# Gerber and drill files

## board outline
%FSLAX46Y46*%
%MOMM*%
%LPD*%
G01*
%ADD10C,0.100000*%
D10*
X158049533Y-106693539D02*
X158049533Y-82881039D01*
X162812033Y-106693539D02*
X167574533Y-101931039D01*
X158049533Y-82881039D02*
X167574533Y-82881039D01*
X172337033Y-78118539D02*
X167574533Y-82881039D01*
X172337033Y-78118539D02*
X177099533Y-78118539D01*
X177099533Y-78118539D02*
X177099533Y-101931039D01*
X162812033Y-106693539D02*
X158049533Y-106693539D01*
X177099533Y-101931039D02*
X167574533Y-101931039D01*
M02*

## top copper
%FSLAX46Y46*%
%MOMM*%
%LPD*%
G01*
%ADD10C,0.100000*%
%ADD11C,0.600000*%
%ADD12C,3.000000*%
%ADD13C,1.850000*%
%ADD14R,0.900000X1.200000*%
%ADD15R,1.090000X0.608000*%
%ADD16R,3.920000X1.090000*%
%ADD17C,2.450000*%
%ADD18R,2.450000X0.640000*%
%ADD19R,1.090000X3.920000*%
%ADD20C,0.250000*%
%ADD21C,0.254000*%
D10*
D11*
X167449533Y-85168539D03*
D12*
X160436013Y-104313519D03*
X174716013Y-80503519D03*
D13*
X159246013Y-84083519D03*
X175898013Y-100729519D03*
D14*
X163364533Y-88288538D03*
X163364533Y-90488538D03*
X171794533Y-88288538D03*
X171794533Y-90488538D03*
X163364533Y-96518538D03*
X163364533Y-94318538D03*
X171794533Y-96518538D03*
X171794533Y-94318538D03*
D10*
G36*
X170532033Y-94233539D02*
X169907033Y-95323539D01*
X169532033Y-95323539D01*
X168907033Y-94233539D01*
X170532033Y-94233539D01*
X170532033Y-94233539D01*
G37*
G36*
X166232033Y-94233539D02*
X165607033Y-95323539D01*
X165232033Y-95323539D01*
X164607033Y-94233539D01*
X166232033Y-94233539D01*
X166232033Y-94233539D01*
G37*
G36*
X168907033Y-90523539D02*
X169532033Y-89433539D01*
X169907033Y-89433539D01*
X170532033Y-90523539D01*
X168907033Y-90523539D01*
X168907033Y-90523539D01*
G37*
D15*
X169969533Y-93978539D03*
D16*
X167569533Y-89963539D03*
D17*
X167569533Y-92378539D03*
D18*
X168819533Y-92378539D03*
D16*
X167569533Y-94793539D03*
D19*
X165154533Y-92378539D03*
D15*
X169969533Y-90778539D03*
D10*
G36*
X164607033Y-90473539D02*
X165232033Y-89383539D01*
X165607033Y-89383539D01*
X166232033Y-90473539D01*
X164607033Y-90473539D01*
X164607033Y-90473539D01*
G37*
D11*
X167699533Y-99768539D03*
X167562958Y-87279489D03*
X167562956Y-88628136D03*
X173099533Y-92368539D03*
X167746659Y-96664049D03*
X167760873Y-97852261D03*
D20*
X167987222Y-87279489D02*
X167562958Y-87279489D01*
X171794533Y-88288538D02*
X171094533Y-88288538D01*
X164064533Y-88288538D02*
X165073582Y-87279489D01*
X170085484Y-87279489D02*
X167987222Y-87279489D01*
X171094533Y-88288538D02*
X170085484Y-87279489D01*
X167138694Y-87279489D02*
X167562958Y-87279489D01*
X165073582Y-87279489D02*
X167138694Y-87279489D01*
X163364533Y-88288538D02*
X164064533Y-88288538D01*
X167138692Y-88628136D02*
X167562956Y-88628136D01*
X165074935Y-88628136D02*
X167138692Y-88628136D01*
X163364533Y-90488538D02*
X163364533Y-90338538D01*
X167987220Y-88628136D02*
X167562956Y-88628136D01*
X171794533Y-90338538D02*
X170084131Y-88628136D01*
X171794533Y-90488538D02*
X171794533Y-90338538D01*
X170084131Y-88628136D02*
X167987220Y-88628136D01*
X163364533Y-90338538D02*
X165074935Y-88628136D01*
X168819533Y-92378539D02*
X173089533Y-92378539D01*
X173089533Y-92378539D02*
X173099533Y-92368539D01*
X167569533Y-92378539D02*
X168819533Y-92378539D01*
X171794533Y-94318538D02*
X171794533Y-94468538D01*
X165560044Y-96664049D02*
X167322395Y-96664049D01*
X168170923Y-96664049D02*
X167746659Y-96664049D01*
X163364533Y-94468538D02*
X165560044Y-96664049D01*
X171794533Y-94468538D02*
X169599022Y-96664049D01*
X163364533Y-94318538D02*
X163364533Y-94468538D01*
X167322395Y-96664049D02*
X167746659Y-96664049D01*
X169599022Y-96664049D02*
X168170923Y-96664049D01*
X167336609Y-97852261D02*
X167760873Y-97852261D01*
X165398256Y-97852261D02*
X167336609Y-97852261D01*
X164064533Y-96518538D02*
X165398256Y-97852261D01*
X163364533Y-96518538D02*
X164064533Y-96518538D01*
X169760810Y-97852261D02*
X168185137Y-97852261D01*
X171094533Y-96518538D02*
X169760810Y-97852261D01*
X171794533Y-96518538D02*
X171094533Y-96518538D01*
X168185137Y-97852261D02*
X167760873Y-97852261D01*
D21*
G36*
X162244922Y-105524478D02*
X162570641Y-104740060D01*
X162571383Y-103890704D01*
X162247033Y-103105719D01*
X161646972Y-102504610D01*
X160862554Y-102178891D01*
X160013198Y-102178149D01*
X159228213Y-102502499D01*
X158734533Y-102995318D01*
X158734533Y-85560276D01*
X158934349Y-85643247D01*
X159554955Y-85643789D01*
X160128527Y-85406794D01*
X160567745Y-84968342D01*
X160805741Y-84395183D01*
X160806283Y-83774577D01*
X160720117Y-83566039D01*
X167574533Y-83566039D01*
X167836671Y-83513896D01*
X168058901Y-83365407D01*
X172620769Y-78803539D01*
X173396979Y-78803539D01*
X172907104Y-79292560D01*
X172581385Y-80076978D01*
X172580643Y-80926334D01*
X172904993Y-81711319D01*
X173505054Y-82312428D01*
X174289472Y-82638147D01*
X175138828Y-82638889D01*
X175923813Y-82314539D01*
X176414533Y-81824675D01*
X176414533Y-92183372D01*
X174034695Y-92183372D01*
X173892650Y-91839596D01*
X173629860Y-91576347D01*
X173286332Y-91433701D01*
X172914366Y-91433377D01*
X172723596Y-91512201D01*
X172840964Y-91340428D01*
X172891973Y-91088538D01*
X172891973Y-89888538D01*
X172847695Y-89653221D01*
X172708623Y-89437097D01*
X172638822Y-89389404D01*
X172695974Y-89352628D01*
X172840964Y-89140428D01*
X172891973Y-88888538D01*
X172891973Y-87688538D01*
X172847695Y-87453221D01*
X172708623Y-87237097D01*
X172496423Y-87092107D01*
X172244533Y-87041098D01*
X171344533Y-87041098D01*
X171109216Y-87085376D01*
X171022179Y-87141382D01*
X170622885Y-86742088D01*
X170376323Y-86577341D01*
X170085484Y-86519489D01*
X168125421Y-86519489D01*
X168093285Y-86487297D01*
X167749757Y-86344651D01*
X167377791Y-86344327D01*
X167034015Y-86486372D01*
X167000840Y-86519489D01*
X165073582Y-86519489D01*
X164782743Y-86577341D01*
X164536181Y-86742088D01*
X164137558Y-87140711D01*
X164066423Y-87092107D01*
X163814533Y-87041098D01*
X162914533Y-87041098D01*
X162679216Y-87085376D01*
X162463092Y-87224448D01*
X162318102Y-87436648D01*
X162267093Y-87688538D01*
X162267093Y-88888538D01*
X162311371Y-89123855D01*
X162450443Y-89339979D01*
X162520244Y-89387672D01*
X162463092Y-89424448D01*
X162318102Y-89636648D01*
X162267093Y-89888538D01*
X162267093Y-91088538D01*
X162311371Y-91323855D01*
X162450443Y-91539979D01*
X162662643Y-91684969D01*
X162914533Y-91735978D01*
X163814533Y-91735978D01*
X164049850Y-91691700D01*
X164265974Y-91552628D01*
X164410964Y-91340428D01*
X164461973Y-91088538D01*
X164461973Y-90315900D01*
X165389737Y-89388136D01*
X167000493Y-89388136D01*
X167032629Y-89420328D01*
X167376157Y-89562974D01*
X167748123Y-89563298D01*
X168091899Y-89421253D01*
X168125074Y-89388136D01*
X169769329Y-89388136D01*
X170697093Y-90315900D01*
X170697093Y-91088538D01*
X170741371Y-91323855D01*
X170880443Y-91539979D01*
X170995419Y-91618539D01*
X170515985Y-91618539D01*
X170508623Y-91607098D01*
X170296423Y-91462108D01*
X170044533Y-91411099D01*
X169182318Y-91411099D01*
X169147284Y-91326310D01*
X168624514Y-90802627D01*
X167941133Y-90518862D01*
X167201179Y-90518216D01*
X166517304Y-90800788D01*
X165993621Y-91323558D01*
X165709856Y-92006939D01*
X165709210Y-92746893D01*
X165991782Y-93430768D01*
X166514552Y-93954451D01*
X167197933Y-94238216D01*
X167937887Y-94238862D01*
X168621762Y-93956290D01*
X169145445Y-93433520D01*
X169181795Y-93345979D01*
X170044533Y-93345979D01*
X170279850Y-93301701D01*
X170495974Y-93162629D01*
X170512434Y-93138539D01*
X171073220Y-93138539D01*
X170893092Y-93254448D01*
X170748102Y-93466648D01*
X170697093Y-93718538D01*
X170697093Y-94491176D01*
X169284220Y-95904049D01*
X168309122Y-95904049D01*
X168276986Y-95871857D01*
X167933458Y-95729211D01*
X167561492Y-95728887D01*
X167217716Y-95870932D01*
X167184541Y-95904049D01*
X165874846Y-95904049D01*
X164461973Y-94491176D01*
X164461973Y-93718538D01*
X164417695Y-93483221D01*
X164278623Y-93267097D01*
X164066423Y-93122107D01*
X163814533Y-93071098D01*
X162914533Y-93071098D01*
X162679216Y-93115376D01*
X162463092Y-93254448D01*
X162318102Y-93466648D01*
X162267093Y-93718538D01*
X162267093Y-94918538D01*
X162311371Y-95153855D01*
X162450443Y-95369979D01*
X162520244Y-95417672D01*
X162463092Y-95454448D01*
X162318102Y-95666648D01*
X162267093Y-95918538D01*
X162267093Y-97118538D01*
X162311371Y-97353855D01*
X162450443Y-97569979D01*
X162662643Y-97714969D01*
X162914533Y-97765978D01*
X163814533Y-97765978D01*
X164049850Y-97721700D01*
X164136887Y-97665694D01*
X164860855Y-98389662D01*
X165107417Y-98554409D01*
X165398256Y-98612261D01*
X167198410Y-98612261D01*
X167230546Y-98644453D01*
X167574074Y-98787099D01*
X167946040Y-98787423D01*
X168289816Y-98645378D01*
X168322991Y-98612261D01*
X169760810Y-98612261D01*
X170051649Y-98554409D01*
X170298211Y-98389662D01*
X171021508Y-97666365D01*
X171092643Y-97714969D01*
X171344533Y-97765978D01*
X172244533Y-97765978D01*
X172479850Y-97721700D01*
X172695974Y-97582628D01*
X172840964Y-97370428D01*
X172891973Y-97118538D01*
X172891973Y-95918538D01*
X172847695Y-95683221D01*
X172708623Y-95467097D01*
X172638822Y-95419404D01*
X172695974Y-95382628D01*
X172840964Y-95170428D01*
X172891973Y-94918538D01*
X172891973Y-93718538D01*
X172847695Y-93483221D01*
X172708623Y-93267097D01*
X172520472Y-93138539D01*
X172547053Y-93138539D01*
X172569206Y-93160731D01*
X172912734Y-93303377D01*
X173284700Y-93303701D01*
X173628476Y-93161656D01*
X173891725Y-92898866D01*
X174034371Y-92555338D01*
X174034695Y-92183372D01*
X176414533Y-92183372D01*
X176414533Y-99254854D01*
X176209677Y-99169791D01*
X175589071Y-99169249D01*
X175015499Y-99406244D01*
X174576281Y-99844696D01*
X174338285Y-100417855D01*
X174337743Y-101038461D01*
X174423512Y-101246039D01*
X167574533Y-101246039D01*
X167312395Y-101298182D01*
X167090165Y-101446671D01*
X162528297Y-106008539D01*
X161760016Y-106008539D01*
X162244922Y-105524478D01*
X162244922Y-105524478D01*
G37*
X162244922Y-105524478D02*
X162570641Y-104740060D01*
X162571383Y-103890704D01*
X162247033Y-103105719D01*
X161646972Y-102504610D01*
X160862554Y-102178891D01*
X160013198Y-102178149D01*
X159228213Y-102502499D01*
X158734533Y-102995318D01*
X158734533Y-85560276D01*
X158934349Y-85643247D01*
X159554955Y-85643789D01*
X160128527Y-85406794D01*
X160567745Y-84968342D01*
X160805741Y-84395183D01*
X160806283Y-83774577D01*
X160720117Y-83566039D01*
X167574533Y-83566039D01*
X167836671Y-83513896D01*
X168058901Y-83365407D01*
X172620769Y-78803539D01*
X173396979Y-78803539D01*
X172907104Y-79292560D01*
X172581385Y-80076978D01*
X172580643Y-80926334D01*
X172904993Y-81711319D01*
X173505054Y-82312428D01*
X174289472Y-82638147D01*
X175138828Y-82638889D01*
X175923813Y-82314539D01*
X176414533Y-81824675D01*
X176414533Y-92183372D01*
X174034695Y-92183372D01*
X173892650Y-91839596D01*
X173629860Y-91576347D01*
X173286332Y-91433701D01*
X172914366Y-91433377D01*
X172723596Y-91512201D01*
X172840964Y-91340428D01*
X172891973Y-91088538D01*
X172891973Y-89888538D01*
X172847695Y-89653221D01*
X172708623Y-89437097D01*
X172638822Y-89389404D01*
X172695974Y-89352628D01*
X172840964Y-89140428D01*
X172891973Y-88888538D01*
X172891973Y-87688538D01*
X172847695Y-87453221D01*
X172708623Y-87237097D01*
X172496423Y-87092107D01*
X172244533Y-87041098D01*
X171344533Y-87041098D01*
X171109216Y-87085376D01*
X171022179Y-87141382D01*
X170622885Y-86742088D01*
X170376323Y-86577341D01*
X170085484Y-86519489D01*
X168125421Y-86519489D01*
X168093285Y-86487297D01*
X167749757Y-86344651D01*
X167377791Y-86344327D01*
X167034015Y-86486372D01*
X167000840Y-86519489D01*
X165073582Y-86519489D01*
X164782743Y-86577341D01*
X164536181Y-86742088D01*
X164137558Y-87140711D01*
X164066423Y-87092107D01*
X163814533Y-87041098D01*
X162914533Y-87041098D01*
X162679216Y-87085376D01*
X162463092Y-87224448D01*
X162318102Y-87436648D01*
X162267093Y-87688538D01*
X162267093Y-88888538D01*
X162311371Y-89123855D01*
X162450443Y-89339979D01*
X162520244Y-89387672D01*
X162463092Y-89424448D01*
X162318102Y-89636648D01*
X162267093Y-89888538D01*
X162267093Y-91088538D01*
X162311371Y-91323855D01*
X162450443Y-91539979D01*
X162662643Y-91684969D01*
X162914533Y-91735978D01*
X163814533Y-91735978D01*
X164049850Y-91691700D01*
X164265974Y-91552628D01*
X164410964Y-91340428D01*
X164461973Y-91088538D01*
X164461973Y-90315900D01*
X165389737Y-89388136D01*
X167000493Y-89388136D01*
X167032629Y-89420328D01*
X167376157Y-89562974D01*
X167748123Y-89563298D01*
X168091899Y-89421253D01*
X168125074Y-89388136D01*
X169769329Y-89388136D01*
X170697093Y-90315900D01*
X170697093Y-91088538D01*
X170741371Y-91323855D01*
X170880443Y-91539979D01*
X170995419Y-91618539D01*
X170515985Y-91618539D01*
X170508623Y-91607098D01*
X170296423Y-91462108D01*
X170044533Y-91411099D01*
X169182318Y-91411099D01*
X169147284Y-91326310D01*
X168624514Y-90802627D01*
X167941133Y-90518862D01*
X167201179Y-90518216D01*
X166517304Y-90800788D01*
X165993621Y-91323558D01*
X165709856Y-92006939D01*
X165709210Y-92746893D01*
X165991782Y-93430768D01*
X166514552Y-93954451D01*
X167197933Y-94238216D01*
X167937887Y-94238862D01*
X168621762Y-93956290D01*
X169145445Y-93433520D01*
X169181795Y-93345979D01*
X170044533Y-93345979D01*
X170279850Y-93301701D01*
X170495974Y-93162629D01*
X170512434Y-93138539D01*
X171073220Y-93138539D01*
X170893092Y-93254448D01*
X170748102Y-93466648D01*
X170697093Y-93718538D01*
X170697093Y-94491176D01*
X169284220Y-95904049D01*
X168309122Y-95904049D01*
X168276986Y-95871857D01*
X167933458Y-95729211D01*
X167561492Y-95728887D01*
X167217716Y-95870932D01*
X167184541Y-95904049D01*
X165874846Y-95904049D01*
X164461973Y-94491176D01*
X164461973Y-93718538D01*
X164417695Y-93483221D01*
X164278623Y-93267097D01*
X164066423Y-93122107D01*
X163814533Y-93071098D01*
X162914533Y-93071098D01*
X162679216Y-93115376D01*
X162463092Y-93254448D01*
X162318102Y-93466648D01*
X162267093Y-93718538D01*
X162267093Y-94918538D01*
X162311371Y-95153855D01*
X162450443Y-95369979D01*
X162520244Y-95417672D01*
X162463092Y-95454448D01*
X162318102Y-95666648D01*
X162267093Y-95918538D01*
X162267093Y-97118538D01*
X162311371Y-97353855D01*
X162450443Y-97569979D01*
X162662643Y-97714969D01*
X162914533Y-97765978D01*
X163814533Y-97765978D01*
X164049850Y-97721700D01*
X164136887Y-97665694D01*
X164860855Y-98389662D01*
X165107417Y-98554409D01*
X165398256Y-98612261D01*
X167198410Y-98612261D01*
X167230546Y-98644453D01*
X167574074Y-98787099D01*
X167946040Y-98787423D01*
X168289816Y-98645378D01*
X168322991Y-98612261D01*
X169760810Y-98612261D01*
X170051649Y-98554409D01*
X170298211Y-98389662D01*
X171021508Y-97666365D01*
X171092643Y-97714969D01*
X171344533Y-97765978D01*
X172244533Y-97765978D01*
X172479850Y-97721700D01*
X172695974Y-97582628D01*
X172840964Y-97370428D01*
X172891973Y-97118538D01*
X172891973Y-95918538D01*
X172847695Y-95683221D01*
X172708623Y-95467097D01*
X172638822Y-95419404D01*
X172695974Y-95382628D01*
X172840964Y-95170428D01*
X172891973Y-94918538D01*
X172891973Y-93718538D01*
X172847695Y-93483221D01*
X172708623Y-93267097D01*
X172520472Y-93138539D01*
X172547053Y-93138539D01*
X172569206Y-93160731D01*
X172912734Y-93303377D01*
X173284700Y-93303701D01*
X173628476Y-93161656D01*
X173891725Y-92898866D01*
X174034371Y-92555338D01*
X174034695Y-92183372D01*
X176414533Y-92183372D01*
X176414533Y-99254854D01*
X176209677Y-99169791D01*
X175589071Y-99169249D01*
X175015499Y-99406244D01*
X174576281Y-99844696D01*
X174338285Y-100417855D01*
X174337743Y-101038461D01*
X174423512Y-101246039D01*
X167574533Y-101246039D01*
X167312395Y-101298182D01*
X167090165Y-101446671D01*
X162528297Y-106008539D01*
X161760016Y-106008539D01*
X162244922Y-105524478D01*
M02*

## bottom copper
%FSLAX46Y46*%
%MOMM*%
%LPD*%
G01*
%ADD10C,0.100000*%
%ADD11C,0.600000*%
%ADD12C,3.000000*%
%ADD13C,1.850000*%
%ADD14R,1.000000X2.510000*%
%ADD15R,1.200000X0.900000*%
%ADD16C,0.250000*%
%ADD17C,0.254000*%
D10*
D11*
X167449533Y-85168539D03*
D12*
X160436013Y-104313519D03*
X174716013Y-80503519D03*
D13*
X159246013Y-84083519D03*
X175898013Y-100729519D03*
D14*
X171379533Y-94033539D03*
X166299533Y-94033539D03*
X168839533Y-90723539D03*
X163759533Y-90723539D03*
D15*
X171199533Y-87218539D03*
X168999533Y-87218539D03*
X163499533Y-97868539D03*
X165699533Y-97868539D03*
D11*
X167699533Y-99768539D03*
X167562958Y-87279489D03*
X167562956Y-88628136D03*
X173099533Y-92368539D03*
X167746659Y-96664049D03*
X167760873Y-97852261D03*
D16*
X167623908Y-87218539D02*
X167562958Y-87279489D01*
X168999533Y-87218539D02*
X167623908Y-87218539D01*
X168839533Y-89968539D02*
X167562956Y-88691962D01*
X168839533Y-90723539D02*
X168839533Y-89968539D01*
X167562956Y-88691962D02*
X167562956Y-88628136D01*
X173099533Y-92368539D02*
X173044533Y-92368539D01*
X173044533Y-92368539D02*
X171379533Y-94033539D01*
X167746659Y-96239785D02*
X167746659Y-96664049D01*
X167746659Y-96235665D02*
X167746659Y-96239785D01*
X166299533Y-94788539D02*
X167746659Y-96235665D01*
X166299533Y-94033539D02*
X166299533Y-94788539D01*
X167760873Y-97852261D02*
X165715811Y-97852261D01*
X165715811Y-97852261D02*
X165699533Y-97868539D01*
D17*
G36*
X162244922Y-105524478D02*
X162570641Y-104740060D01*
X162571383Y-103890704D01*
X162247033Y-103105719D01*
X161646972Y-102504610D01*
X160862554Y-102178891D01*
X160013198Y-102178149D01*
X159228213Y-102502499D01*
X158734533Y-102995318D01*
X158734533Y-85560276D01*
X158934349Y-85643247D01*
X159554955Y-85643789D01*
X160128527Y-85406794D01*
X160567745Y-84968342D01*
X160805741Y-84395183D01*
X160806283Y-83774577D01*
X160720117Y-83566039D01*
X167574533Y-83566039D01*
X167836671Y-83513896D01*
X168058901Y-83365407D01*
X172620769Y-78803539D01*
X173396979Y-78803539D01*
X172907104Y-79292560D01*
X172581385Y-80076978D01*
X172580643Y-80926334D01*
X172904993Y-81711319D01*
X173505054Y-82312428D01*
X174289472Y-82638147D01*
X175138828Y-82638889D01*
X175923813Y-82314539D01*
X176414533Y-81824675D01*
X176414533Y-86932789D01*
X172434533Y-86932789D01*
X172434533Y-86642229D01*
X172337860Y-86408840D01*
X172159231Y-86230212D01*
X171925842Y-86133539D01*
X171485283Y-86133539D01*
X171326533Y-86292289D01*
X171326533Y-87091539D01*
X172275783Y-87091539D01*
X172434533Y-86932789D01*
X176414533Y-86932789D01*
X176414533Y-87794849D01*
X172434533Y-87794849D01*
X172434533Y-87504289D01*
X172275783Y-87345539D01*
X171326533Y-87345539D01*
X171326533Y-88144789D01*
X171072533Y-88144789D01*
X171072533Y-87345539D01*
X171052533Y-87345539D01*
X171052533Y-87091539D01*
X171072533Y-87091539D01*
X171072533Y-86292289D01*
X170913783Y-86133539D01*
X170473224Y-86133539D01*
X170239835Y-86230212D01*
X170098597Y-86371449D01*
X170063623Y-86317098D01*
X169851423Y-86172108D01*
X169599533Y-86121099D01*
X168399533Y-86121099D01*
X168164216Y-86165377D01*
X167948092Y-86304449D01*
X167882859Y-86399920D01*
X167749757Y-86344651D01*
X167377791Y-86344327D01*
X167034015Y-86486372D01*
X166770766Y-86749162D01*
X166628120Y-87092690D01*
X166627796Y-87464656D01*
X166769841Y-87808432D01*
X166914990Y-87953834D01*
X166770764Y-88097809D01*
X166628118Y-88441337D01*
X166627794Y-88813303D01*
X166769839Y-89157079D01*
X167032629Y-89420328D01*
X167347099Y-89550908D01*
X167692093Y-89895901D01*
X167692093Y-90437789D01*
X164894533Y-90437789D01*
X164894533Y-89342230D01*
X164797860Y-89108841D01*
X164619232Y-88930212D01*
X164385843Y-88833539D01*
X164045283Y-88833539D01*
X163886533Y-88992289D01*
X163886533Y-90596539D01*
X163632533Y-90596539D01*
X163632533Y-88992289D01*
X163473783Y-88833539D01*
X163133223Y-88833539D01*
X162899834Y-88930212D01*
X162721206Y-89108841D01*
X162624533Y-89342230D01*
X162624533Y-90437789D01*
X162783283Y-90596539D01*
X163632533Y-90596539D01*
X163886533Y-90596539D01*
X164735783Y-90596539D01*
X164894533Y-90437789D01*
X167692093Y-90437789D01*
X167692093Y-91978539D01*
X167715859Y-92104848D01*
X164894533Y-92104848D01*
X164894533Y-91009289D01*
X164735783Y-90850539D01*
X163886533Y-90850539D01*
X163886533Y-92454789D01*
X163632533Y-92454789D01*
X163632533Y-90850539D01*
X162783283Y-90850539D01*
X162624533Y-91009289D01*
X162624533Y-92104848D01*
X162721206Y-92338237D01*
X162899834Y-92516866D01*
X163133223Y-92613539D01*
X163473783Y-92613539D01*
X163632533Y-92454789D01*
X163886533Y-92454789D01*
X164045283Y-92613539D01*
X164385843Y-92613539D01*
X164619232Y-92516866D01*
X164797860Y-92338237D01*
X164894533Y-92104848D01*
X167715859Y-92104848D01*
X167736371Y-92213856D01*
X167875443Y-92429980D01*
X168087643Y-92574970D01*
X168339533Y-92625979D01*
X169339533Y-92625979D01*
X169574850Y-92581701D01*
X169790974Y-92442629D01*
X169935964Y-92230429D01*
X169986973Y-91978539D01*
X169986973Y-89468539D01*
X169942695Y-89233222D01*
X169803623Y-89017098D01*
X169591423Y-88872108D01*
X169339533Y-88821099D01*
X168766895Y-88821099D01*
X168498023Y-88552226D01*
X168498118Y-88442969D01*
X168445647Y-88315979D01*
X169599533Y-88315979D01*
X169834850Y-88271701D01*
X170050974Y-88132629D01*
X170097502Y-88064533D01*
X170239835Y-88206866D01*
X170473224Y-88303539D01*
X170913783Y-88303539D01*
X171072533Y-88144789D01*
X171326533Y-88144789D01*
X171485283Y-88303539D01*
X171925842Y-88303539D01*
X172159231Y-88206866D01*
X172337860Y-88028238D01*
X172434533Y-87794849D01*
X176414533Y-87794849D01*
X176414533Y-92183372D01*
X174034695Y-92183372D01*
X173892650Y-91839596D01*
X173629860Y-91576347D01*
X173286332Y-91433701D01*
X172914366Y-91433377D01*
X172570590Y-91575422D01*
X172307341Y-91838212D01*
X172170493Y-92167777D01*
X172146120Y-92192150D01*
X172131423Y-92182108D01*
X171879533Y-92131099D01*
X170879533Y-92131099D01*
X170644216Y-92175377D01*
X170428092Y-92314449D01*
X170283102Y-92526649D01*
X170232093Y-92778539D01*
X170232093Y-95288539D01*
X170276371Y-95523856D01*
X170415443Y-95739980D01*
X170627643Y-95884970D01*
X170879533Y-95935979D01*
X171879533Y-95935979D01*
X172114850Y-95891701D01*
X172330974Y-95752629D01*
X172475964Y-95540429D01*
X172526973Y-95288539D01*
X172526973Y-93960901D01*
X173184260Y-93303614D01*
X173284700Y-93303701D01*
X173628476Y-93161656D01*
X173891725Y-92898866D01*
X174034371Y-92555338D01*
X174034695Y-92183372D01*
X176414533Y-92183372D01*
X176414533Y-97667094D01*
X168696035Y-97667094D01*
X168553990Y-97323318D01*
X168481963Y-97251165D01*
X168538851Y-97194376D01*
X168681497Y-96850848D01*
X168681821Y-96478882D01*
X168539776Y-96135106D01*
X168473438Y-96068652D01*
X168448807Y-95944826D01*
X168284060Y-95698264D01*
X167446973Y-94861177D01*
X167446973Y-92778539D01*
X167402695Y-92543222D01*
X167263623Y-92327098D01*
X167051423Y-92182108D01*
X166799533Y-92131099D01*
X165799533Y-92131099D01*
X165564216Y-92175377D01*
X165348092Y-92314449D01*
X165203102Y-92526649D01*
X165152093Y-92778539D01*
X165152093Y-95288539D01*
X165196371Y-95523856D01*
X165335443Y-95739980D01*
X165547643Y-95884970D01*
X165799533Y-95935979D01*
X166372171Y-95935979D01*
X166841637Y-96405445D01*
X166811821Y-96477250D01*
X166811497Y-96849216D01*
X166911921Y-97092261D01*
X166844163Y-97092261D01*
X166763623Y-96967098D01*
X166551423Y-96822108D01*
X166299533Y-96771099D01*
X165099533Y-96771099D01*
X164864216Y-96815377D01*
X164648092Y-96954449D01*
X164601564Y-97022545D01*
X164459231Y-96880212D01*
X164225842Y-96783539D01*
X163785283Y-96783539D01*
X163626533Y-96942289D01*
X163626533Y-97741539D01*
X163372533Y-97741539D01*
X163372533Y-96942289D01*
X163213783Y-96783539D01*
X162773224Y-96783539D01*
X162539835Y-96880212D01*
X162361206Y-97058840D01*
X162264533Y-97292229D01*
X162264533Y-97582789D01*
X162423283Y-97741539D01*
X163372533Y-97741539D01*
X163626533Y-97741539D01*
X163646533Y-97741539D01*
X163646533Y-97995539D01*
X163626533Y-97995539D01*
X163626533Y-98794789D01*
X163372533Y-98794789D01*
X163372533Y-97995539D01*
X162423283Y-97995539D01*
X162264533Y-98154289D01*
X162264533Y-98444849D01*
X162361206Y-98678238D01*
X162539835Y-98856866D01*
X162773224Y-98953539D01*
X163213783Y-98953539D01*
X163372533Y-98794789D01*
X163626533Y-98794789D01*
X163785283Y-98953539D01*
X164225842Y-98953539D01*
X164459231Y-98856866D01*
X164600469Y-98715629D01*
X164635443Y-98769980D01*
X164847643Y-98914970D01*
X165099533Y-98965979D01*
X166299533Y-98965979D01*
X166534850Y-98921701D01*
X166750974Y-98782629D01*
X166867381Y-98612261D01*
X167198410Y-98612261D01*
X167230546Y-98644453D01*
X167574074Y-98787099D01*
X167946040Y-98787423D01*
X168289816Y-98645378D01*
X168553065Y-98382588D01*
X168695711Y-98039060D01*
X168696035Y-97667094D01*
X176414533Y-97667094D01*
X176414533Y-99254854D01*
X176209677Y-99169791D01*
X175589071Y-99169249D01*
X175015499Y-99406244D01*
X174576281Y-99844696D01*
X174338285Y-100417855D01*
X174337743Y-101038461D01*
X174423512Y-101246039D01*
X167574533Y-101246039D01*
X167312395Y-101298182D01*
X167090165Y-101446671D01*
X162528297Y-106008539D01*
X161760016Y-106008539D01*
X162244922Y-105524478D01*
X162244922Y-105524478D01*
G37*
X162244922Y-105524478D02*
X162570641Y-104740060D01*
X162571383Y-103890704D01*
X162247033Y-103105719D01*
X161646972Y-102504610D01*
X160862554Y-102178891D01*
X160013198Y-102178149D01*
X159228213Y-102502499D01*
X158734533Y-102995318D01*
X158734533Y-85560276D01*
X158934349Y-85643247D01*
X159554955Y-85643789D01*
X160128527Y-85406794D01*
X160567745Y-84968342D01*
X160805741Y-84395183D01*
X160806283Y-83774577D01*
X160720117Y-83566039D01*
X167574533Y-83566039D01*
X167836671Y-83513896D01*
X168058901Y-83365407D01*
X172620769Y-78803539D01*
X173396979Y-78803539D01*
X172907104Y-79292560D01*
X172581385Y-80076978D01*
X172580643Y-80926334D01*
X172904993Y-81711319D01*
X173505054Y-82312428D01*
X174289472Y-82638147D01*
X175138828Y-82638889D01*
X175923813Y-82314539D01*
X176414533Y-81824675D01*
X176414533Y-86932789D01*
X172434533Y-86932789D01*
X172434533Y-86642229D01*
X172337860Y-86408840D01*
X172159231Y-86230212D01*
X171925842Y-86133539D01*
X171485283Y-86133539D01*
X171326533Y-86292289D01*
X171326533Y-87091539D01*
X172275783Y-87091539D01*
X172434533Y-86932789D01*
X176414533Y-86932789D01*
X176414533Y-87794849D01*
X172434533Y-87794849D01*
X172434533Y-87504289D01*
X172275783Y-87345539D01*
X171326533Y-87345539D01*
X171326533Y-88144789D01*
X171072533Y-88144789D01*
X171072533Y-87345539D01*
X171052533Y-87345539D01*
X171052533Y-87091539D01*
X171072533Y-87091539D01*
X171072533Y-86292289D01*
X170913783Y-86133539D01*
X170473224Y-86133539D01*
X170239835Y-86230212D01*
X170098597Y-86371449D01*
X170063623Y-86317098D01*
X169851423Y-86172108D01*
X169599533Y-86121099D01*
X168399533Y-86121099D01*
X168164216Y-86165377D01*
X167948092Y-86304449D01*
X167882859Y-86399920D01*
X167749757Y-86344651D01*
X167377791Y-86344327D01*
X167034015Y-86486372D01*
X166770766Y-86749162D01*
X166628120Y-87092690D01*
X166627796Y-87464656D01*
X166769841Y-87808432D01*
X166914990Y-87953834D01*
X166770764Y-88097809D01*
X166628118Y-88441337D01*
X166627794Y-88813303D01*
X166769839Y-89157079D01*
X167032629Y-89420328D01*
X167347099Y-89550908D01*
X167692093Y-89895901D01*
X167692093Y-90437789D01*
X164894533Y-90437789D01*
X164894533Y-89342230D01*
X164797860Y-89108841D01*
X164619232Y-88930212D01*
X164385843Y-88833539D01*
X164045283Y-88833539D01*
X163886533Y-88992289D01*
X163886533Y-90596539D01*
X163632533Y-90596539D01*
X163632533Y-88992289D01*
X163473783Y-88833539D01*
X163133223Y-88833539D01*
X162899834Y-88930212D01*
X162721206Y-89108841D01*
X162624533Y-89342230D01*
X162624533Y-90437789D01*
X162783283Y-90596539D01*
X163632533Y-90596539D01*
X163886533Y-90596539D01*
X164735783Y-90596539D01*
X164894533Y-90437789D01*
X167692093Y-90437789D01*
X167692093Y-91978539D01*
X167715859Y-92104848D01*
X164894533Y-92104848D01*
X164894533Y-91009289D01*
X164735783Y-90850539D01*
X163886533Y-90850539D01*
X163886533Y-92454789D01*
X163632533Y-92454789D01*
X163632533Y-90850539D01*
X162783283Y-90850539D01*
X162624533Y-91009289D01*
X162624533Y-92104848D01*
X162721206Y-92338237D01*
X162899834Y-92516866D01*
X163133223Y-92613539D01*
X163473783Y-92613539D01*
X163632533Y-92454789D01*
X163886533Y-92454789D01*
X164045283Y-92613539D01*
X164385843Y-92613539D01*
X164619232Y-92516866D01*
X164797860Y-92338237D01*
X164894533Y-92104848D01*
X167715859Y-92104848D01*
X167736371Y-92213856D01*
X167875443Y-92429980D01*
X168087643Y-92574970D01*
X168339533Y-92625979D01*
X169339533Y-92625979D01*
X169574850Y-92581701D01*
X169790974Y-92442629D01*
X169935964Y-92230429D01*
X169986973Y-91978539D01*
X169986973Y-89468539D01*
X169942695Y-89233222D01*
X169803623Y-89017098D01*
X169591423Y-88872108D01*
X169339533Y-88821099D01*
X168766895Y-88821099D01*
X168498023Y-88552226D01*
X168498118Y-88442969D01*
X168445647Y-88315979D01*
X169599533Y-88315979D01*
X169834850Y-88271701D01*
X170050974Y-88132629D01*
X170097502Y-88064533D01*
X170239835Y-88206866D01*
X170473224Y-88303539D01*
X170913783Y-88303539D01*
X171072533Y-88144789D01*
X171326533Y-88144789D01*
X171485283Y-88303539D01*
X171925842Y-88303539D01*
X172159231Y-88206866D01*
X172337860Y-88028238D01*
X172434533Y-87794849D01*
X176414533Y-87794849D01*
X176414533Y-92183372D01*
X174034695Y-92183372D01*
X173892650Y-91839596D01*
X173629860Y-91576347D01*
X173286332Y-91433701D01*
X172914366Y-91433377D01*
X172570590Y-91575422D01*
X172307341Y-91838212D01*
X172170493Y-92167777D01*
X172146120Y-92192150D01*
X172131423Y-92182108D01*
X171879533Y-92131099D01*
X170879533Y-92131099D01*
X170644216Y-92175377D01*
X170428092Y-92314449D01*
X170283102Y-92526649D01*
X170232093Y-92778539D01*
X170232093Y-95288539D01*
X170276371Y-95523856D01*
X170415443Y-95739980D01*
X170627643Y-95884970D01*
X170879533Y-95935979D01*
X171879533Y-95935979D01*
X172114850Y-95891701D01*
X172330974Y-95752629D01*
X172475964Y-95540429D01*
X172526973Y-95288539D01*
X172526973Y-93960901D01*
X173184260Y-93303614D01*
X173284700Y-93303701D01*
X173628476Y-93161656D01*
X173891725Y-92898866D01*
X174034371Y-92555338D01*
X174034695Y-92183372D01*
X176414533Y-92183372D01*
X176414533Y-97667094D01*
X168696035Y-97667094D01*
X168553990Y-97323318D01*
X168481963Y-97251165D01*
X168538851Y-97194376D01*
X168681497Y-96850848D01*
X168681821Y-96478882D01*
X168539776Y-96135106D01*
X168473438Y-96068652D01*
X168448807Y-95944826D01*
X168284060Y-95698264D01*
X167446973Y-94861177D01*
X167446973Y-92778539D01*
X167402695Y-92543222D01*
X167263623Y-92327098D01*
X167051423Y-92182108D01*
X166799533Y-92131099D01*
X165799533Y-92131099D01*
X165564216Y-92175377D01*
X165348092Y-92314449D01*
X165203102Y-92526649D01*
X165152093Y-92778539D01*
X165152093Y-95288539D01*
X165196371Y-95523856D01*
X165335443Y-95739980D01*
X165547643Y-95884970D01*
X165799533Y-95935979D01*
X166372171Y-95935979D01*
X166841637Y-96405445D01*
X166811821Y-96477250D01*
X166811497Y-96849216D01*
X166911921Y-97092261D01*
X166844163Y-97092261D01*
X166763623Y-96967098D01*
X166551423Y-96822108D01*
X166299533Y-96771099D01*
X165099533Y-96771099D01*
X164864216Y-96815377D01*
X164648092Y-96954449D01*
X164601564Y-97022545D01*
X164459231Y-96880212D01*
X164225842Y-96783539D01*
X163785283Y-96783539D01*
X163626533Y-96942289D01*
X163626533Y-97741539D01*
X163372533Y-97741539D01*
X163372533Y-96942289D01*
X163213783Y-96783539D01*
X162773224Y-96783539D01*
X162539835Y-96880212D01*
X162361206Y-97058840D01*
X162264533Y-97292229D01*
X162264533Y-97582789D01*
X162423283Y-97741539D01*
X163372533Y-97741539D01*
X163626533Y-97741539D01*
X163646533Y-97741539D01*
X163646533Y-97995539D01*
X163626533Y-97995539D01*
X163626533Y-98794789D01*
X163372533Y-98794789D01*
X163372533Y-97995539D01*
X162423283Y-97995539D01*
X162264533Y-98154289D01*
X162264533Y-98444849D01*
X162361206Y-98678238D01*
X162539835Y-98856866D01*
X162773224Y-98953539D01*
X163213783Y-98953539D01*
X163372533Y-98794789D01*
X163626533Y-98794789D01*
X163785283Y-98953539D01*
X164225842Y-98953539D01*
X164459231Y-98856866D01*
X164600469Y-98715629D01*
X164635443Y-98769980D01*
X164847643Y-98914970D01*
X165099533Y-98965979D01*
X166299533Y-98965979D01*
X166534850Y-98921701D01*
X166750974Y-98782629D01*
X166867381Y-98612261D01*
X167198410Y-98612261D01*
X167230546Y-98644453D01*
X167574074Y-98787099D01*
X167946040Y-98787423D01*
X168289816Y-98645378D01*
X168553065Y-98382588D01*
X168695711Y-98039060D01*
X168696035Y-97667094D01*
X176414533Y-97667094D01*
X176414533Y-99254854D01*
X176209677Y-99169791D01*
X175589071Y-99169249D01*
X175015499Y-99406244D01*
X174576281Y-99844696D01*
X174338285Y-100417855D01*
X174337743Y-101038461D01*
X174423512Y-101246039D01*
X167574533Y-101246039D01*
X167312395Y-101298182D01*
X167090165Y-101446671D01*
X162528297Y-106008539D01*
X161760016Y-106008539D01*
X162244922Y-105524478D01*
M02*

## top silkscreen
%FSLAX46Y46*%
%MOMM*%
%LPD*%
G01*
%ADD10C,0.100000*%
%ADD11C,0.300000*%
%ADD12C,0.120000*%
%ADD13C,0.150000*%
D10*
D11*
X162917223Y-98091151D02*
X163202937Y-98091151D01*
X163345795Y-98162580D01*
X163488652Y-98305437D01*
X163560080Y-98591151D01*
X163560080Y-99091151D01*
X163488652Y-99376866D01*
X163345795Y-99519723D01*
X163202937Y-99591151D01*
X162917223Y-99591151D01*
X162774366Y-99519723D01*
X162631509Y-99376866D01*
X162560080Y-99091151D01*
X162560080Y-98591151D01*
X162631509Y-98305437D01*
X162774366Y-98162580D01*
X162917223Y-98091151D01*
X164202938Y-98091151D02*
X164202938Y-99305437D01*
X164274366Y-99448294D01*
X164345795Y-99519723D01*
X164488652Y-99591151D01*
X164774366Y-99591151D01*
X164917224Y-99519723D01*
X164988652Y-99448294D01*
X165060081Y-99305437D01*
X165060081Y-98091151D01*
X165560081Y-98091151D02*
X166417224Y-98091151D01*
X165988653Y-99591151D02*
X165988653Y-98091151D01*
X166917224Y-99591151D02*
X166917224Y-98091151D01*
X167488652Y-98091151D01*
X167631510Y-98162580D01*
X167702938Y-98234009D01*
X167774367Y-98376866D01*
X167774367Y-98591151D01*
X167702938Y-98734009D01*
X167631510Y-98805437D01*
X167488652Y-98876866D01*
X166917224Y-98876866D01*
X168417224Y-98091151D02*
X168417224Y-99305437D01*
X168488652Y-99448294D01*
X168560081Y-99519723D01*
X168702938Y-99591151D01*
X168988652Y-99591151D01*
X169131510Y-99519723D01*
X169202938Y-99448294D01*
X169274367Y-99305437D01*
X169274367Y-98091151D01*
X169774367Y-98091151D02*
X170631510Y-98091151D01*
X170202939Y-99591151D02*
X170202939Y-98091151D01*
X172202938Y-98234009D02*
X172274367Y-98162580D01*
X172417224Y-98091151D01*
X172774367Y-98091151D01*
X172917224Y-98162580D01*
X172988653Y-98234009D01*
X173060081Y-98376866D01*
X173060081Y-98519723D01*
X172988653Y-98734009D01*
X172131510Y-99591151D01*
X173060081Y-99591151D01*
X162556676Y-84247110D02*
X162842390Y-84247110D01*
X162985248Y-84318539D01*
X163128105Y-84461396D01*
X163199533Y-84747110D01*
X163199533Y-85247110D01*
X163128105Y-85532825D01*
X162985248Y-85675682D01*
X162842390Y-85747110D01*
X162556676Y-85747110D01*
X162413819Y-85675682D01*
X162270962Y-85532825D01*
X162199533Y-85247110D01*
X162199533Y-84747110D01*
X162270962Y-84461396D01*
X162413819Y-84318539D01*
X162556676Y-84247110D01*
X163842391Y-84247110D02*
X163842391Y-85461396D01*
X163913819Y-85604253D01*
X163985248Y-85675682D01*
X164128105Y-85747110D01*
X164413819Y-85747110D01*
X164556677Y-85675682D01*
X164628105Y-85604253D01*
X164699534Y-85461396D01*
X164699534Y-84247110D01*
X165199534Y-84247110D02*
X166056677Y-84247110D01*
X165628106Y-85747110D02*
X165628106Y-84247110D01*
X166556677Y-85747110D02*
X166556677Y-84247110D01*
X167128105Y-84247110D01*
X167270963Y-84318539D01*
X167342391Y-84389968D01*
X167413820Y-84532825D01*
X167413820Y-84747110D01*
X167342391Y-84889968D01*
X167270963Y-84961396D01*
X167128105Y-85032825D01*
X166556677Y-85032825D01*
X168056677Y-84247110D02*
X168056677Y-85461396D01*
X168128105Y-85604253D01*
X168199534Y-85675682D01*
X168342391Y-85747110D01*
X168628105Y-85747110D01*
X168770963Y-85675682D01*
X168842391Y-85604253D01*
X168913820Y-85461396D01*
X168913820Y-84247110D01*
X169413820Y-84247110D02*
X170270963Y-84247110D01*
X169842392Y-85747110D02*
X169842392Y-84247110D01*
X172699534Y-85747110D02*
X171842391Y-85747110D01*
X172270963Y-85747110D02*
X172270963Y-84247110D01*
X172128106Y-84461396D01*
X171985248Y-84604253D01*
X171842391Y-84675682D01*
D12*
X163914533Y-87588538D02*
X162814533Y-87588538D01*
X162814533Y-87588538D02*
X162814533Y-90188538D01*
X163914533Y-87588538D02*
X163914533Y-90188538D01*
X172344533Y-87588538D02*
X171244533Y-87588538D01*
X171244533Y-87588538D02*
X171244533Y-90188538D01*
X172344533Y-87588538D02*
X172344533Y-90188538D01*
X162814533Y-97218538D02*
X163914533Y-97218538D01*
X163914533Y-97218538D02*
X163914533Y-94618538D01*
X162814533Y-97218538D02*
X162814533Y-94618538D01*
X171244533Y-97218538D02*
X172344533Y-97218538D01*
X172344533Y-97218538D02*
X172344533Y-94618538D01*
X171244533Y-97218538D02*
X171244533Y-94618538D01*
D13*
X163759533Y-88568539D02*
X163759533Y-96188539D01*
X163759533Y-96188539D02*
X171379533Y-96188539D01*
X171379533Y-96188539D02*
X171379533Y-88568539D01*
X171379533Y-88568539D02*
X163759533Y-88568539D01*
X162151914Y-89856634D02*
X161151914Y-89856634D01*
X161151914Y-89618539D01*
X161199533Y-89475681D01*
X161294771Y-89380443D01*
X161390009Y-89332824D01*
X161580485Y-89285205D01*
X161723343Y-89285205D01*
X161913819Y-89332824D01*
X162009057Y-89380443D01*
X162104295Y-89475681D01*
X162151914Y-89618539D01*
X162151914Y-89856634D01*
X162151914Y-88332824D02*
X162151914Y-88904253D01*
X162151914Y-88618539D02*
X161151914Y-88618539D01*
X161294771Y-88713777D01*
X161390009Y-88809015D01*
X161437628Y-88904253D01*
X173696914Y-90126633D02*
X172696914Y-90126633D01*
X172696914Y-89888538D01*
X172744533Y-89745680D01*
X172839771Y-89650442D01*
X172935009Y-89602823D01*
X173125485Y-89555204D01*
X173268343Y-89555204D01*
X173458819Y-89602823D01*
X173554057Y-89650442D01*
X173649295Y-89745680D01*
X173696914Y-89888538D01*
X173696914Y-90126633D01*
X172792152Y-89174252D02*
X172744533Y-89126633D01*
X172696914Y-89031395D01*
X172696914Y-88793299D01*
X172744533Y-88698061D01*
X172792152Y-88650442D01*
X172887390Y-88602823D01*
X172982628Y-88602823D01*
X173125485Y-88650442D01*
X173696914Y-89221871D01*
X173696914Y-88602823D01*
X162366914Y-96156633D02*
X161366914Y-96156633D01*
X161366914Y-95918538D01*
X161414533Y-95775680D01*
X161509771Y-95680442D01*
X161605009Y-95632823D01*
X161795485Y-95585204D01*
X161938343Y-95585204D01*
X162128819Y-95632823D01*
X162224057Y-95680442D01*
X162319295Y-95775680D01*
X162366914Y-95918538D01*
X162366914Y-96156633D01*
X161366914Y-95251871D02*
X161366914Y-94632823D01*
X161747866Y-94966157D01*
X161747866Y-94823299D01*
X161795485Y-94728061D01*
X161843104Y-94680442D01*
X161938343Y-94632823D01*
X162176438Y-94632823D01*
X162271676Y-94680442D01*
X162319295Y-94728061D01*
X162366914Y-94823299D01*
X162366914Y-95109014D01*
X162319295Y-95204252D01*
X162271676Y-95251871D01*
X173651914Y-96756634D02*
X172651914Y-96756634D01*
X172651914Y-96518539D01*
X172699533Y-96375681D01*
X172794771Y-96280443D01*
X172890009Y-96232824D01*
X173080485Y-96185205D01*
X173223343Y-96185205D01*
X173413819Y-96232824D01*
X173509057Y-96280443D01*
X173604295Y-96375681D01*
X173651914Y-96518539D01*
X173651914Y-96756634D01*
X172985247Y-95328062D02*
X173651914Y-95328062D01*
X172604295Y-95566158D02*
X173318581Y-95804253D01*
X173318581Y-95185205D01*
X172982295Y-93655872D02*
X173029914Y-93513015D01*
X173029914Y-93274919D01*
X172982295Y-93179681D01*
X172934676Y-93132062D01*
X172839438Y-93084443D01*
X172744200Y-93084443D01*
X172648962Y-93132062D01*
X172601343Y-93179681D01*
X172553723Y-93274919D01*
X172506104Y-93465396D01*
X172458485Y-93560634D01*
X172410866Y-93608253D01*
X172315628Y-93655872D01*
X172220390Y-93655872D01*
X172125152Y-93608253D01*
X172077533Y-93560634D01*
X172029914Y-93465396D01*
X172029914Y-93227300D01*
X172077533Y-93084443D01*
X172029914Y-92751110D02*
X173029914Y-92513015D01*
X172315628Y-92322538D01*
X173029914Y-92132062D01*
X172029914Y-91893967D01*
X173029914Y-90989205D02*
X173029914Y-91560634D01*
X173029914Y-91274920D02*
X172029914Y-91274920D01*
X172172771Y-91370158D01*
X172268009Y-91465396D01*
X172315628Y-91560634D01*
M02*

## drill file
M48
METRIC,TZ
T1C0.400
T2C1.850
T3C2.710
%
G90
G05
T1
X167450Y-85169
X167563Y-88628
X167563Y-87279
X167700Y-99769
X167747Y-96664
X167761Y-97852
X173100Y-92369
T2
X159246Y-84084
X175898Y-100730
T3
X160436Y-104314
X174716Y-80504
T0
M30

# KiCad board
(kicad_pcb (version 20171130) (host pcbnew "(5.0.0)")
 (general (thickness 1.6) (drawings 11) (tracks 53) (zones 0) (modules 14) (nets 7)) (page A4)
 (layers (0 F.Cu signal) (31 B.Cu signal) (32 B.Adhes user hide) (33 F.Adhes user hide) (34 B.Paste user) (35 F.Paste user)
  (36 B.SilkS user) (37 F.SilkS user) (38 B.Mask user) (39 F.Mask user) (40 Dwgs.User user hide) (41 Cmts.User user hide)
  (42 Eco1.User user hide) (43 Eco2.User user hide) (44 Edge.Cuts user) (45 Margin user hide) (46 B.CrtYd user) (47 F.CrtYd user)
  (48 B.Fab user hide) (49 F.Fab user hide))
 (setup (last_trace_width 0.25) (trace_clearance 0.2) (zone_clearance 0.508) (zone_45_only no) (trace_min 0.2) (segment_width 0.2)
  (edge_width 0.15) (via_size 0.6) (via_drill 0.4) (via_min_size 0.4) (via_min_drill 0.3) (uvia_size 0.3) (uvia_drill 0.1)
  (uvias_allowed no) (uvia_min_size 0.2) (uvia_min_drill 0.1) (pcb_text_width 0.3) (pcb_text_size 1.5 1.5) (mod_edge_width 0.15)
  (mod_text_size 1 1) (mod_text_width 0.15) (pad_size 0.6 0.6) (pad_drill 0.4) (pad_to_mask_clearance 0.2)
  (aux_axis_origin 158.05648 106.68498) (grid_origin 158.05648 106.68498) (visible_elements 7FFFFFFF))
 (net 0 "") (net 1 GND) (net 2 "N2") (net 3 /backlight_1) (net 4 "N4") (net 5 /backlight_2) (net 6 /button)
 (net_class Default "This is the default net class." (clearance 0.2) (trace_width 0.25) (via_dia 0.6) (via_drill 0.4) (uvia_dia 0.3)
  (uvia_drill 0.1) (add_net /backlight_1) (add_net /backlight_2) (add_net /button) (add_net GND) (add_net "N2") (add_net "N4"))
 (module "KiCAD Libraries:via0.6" (layer F.Cu) (at 167.449533 85.168539 180) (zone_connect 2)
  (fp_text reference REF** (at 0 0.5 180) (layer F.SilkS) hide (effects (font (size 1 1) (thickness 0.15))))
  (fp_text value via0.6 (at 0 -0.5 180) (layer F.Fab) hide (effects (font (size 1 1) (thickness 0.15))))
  (pad 1 thru_hole circle (at 0 0 180) (size 0.6 0.6) (drill 0.4) (layers *.Cu) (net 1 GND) (zone_connect 2)))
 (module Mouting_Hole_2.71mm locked (layer F.Cu) (at 160.436013 104.313519 180)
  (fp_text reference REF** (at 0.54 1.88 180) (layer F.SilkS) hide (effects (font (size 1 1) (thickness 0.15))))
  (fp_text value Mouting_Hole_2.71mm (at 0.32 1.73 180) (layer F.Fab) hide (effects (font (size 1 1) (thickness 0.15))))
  (pad 1 thru_hole circle (at 0 0 180) (size 3 3) (drill 2.71) (layers *.Cu) (clearance 0.5) (zone_connect 0)))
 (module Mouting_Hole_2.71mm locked (layer F.Cu) (at 174.716013 80.503519 180)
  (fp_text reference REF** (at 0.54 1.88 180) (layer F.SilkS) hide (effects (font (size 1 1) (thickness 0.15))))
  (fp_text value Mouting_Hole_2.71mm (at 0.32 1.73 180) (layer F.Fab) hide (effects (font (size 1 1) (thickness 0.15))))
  (pad 1 thru_hole circle (at 0 0 180) (size 3 3) (drill 2.71) (layers *.Cu) (clearance 0.5) (zone_connect 0)))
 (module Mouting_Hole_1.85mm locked (layer F.Cu) (at 159.246013 84.083519 180)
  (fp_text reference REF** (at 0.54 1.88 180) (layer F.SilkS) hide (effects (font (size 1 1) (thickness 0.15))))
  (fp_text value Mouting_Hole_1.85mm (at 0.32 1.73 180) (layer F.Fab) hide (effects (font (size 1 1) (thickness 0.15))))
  (pad 1 thru_hole circle (at 0 0 180) (size 1.85 1.85) (drill 1.85) (layers *.Cu) (clearance 0.5) (zone_connect 0)))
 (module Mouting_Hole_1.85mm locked (layer F.Cu) (at 175.898013 100.729519 180)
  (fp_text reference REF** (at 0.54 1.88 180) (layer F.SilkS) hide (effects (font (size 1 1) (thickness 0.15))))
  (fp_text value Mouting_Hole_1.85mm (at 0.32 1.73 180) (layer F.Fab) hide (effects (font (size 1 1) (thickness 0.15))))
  (pad 1 thru_hole circle (at 0 0 180) (size 1.85 1.85) (drill 1.85) (layers *.Cu) (clearance 0.5) (zone_connect 0)))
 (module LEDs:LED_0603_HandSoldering (layer F.Cu) (at 163.364533 89.388538 270)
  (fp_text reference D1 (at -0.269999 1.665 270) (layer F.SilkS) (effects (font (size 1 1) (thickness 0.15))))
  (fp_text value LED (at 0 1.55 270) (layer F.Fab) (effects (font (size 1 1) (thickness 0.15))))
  (fp_line (start -1.8 -0.55) (end -1.8 0.55) (layer F.SilkS) (width 0.12))
  (fp_line (start -1.8 0.55) (end 0.8 0.55) (layer F.SilkS) (width 0.12))
  (fp_line (start -1.8 -0.55) (end 0.8 -0.55) (layer F.SilkS) (width 0.12))
  (pad 1 smd rect (at -1.1 0 270) (size 1.2 0.9) (layers F.Cu F.Paste F.Mask) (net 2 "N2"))
  (pad 2 smd rect (at 1.1 0 270) (size 1.2 0.9) (layers F.Cu F.Paste F.Mask) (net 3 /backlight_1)))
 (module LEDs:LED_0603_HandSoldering (layer F.Cu) (at 171.794533 89.388538 270)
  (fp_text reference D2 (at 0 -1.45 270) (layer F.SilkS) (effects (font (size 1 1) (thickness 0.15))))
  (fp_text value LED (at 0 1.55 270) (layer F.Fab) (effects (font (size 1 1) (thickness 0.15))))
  (fp_line (start -1.8 -0.55) (end -1.8 0.55) (layer F.SilkS) (width 0.12))
  (fp_line (start -1.8 0.55) (end 0.8 0.55) (layer F.SilkS) (width 0.12))
  (fp_line (start -1.8 -0.55) (end 0.8 -0.55) (layer F.SilkS) (width 0.12))
  (pad 1 smd rect (at -1.1 0 270) (size 1.2 0.9) (layers F.Cu F.Paste F.Mask) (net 2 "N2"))
  (pad 2 smd rect (at 1.1 0 270) (size 1.2 0.9) (layers F.Cu F.Paste F.Mask) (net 3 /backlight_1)))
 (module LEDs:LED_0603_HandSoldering (layer F.Cu) (at 163.364533 95.418538 90)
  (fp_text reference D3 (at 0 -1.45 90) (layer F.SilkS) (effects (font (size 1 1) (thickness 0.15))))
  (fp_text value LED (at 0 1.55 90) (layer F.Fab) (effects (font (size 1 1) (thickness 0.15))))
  (fp_line (start -1.8 -0.55) (end -1.8 0.55) (layer F.SilkS) (width 0.12))
  (fp_line (start -1.8 0.55) (end 0.8 0.55) (layer F.SilkS) (width 0.12))
  (fp_line (start -1.8 -0.55) (end 0.8 -0.55) (layer F.SilkS) (width 0.12))
  (pad 1 smd rect (at -1.1 0 90) (size 1.2 0.9) (layers F.Cu F.Paste F.Mask) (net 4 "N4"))
  (pad 2 smd rect (at 1.1 0 90) (size 1.2 0.9) (layers F.Cu F.Paste F.Mask) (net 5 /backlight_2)))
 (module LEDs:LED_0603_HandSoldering (layer F.Cu) (at 171.794533 95.418538 90)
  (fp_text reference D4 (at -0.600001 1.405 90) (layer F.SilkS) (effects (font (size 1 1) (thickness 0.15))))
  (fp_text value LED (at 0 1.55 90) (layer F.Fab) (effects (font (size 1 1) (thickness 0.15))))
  (fp_line (start -1.8 -0.55) (end -1.8 0.55) (layer F.SilkS) (width 0.12))
  (fp_line (start -1.8 0.55) (end 0.8 0.55) (layer F.SilkS) (width 0.12))
  (fp_line (start -1.8 -0.55) (end 0.8 -0.55) (layer F.SilkS) (width 0.12))
  (pad 1 smd rect (at -1.1 0 90) (size 1.2 0.9) (layers F.Cu F.Paste F.Mask) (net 4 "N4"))
  (pad 2 smd rect (at 1.1 0 90) (size 1.2 0.9) (layers F.Cu F.Paste F.Mask) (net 5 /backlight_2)))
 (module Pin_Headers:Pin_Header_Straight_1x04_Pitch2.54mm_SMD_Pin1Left (layer B.Cu) (at 167.569533 92.378539 90)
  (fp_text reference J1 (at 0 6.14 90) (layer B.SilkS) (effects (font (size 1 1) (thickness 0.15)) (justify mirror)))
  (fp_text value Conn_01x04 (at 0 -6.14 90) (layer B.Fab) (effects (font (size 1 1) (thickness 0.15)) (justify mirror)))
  (pad 1 smd rect (at -1.655 3.81 90) (size 2.51 1) (layers B.Cu B.Paste B.Mask) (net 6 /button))
  (pad 3 smd rect (at -1.655 -1.27 90) (size 2.51 1) (layers B.Cu B.Paste B.Mask) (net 5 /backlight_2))
  (pad 2 smd rect (at 1.655 1.27 90) (size 2.51 1) (layers B.Cu B.Paste B.Mask) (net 3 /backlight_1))
  (pad 4 smd rect (at 1.655 -3.81 90) (size 2.51 1) (layers B.Cu B.Paste B.Mask) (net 1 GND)))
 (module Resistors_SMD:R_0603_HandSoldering (layer B.Cu) (at 170.099533 87.218539 180)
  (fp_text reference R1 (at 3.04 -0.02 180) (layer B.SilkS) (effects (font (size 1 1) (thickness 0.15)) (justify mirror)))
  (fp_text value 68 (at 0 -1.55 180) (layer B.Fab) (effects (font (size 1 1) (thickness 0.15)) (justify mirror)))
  (pad 1 smd rect (at -1.1 0 180) (size 1.2 0.9) (layers B.Cu B.Paste B.Mask) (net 1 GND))
  (pad 2 smd rect (at 1.1 0 180) (size 1.2 0.9) (layers B.Cu B.Paste B.Mask) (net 2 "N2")))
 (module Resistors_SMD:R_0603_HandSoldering (layer B.Cu) (at 164.599533 97.868539)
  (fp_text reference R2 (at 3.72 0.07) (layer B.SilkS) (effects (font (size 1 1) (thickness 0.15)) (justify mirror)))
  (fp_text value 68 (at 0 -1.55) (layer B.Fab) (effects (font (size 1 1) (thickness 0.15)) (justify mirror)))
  (pad 1 smd rect (at -1.1 0) (size 1.2 0.9) (layers B.Cu B.Paste B.Mask) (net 1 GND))
  (pad 2 smd rect (at 1.1 0) (size 1.2 0.9) (layers B.Cu B.Paste B.Mask) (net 4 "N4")))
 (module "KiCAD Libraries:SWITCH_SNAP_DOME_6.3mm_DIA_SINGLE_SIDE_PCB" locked (layer F.Cu) (at 167.569533 92.378539) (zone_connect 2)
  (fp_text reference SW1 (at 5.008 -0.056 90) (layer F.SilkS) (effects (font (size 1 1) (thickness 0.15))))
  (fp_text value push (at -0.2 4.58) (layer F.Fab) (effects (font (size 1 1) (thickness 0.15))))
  (fp_line (start -3.81 -3.81) (end -3.81 3.81) (layer F.SilkS) (width 0.15))
  (fp_line (start -3.81 3.81) (end 3.81 3.81) (layer F.SilkS) (width 0.15))
  (fp_line (start 3.81 3.81) (end 3.81 -3.81) (layer F.SilkS) (width 0.15))
  (fp_line (start 3.81 -3.81) (end -3.81 -3.81) (layer F.SilkS) (width 0.15))
  (pad 2 smd trapezoid (at 2.15 2.4 180) (size 1 1.09) (rect_delta 0 0.625) (layers F.Cu F.Paste F.Mask) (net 1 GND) (zone_connect 2))
  (pad 2 smd trapezoid (at -2.15 2.4 180) (size 1 1.09) (rect_delta 0 0.625) (layers F.Cu F.Paste F.Mask) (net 1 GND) (zone_connect 2))
  (pad 2 smd trapezoid (at 2.15 -2.4) (size 1 1.09) (rect_delta 0 0.625) (layers F.Cu F.Paste F.Mask) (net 1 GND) (zone_connect 2))
  (pad 2 smd rect (at 2.4 1.6) (size 1.09 0.608) (layers F.Cu F.Paste F.Mask) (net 1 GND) (zone_connect 2))
  (pad 2 smd rect (at 0 -2.415) (size 3.92 1.09) (layers F.Cu F.Paste F.Mask) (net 1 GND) (zone_connect 2))
  (pad 1 smd circle (at 0 0) (size 2.45 2.45) (layers F.Cu F.Paste F.Mask) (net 6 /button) (zone_connect 2))
  (pad 1 smd rect (at 1.25 0) (size 2.45 0.64) (layers F.Cu F.Paste F.Mask) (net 6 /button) (zone_connect 2))
  (pad 2 smd rect (at 0 2.415) (size 3.92 1.09) (layers F.Cu F.Paste F.Mask) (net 1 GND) (zone_connect 2))
  (pad 2 smd rect (at -2.415 0) (size 1.09 3.92) (layers F.Cu F.Paste F.Mask) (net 1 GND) (zone_connect 2))
  (pad 2 smd rect (at 2.4 -1.6) (size 1.09 0.608) (layers F.Cu F.Paste F.Mask) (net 1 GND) (zone_connect 2))
  (pad 2 smd trapezoid (at -2.15 -2.45) (size 1 1.09) (rect_delta 0 0.625) (layers F.Cu F.Paste F.Mask) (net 1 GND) (zone_connect 2)))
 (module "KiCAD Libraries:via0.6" (layer F.Cu) (at 167.699533 99.768539 180) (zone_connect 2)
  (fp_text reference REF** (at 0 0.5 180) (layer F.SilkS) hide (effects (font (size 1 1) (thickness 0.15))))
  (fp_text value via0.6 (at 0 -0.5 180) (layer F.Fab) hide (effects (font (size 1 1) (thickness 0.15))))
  (pad 1 thru_hole circle (at 0 0 180) (size 0.6 0.6) (drill 0.4) (layers *.Cu) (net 1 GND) (zone_connect 2)))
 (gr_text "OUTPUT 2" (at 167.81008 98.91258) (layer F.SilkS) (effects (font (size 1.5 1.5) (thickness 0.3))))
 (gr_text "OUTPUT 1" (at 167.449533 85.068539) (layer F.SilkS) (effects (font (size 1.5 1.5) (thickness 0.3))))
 (gr_line (start 158.049533 106.693539) (end 158.049533 82.881039) (layer Edge.Cuts) (width 0.1))
 (gr_line (start 162.812033 106.693539) (end 167.574533 101.931039) (layer Edge.Cuts) (width 0.1))
 (gr_line (start 158.049533 82.881039) (end 167.574533 82.881039) (layer Edge.Cuts) (width 0.1))
 (gr_line (start 172.337033 78.118539) (end 167.574533 82.881039) (layer Edge.Cuts) (width 0.1))
 (gr_line (start 172.337033 78.118539) (end 177.099533 78.118539) (layer Edge.Cuts) (width 0.1))
 (gr_line (start 177.099533 78.118539) (end 177.099533 101.931039) (layer Edge.Cuts) (width 0.1))
 (gr_line (start 162.812033 106.693539) (end 158.049533 106.693539) (layer Edge.Cuts) (width 0.1))
 (gr_line (start 177.099533 101.931039) (end 167.574533 101.931039) (layer Edge.Cuts) (width 0.1))
 (segment (start 167.623908 87.218539) (end 167.562958 87.279489) (width 0.25) (layer B.Cu) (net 2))
 (segment (start 167.987222 87.279489) (end 167.562958 87.279489) (width 0.25) (layer F.Cu) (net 2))
 (segment (start 168.999533 87.218539) (end 167.623908 87.218539) (width 0.25) (layer B.Cu) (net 2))
 (segment (start 171.794533 88.288538) (end 171.094533 88.288538) (width 0.25) (layer F.Cu) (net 2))
 (segment (start 164.064533 88.288538) (end 165.073582 87.279489) (width 0.25) (layer F.Cu) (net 2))
 (segment (start 170.085484 87.279489) (end 167.987222 87.279489) (width 0.25) (layer F.Cu) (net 2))
 (segment (start 171.094533 88.288538) (end 170.085484 87.279489) (width 0.25) (layer F.Cu) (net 2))
 (segment (start 167.138694 87.279489) (end 167.562958 87.279489) (width 0.25) (layer F.Cu) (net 2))
 (segment (start 165.073582 87.279489) (end 167.138694 87.279489) (width 0.25) (layer F.Cu) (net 2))
 (segment (start 163.364533 88.288538) (end 164.064533 88.288538) (width 0.25) (layer F.Cu) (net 2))
 (via (at 167.562958 87.279489) (size 0.6) (drill 0.4) (layers F.Cu B.Cu) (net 2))
 (segment (start 167.138692 88.628136) (end 167.562956 88.628136) (width 0.25) (layer F.Cu) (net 3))
 (segment (start 168.839533 89.968539) (end 167.562956 88.691962) (width 0.25) (layer B.Cu) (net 3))
 (segment (start 165.074935 88.628136) (end 167.138692 88.628136) (width 0.25) (layer F.Cu) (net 3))
 (segment (start 163.364533 90.488538) (end 163.364533 90.338538) (width 0.25) (layer F.Cu) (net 3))
 (segment (start 167.98722 88.628136) (end 167.562956 88.628136) (width 0.25) (layer F.Cu) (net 3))
 (segment (start 171.794533 90.338538) (end 170.084131 88.628136) (width 0.25) (layer F.Cu) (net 3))
 (segment (start 171.794533 90.488538) (end 171.794533 90.338538) (width 0.25) (layer F.Cu) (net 3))
 (segment (start 168.839533 90.723539) (end 168.839533 89.968539) (width 0.25) (layer B.Cu) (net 3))
 (segment (start 170.084131 88.628136) (end 167.98722 88.628136) (width 0.25) (layer F.Cu) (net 3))
 (segment (start 167.562956 88.691962) (end 167.562956 88.628136) (width 0.25) (layer B.Cu) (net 3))
 (segment (start 163.364533 90.338538) (end 165.074935 88.628136) (width 0.25) (layer F.Cu) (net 3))
 (via (at 167.562956 88.628136) (size 0.6) (drill 0.4) (layers F.Cu B.Cu) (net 3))
 (segment (start 173.099533 92.368539) (end 173.044533 92.368539) (width 0.25) (layer B.Cu) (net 6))
 (segment (start 173.044533 92.368539) (end 171.379533 94.033539) (width 0.25) (layer B.Cu) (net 6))
 (segment (start 168.819533 92.378539) (end 173.089533 92.378539) (width 0.25) (layer F.Cu) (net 6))
 (segment (start 173.089533 92.378539) (end 173.099533 92.368539) (width 0.25) (layer F.Cu) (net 6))
 (via (at 173.099533 92.368539) (size 0.6) (drill 0.4) (layers F.Cu B.Cu) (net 6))
 (segment (start 167.569533 92.378539) (end 168.819533 92.378539) (width 0.25) (layer F.Cu) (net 6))
 (via (at 167.746659 96.664049) (size 0.6) (drill 0.4) (layers F.Cu B.Cu) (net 5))
 (segment (start 171.794533 94.318538) (end 171.794533 94.468538) (width 0.25) (layer F.Cu) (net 5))
 (segment (start 165.560044 96.664049) (end 167.322395 96.664049) (width 0.25) (layer F.Cu) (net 5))
 (segment (start 168.170923 96.664049) (end 167.746659 96.664049) (width 0.25) (layer F.Cu) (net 5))
 (segment (start 163.364533 94.468538) (end 165.560044 96.664049) (width 0.25) (layer F.Cu) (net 5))
 (segment (start 171.794533 94.468538) (end 169.599022 96.664049) (width 0.25) (layer F.Cu) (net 5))
 (segment (start 163.364533 94.318538) (end 163.364533 94.468538) (width 0.25) (layer F.Cu) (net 5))
 (segment (start 167.746659 96.239785) (end 167.746659 96.664049) (width 0.25) (layer B.Cu) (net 5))
 (segment (start 167.746659 96.235665) (end 167.746659 96.239785) (width 0.25) (layer B.Cu) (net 5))
 (segment (start 167.322395 96.664049) (end 167.746659 96.664049) (width 0.25) (layer F.Cu) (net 5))
 (segment (start 166.299533 94.788539) (end 167.746659 96.235665) (width 0.25) (layer B.Cu) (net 5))
 (segment (start 169.599022 96.664049) (end 168.170923 96.664049) (width 0.25) (layer F.Cu) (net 5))
 (segment (start 166.299533 94.033539) (end 166.299533 94.788539) (width 0.25) (layer B.Cu) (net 5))
 (segment (start 167.760873 97.852261) (end 165.715811 97.852261) (width 0.25) (layer B.Cu) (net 4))
 (segment (start 165.715811 97.852261) (end 165.699533 97.868539) (width 0.25) (layer B.Cu) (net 4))
 (segment (start 167.336609 97.852261) (end 167.760873 97.852261) (width 0.25) (layer F.Cu) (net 4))
 (segment (start 165.398256 97.852261) (end 167.336609 97.852261) (width 0.25) (layer F.Cu) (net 4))
 (segment (start 164.064533 96.518538) (end 165.398256 97.852261) (width 0.25) (layer F.Cu) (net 4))
 (segment (start 163.364533 96.518538) (end 164.064533 96.518538) (width 0.25) (layer F.Cu) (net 4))
 (segment (start 169.76081 97.852261) (end 168.185137 97.852261) (width 0.25) (layer F.Cu) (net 4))
 (segment (start 171.094533 96.518538) (end 169.76081 97.852261) (width 0.25) (layer F.Cu) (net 4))
 (segment (start 171.794533 96.518538) (end 171.094533 96.518538) (width 0.25) (layer F.Cu) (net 4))
 (segment (start 168.185137 97.852261) (end 167.760873 97.852261) (width 0.25) (layer F.Cu) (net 4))
 (via (at 167.760873 97.852261) (size 0.6) (drill 0.4) (layers F.Cu B.Cu) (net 4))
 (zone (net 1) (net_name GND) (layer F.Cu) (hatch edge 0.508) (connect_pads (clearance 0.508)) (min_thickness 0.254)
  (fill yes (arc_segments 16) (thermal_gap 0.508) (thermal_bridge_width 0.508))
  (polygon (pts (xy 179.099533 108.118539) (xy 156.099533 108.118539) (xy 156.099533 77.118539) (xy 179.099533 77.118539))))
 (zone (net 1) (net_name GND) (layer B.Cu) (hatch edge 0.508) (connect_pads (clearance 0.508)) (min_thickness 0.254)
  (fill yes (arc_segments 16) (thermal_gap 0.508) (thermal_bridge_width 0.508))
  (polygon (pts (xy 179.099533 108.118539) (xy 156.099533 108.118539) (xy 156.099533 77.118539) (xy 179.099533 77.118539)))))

